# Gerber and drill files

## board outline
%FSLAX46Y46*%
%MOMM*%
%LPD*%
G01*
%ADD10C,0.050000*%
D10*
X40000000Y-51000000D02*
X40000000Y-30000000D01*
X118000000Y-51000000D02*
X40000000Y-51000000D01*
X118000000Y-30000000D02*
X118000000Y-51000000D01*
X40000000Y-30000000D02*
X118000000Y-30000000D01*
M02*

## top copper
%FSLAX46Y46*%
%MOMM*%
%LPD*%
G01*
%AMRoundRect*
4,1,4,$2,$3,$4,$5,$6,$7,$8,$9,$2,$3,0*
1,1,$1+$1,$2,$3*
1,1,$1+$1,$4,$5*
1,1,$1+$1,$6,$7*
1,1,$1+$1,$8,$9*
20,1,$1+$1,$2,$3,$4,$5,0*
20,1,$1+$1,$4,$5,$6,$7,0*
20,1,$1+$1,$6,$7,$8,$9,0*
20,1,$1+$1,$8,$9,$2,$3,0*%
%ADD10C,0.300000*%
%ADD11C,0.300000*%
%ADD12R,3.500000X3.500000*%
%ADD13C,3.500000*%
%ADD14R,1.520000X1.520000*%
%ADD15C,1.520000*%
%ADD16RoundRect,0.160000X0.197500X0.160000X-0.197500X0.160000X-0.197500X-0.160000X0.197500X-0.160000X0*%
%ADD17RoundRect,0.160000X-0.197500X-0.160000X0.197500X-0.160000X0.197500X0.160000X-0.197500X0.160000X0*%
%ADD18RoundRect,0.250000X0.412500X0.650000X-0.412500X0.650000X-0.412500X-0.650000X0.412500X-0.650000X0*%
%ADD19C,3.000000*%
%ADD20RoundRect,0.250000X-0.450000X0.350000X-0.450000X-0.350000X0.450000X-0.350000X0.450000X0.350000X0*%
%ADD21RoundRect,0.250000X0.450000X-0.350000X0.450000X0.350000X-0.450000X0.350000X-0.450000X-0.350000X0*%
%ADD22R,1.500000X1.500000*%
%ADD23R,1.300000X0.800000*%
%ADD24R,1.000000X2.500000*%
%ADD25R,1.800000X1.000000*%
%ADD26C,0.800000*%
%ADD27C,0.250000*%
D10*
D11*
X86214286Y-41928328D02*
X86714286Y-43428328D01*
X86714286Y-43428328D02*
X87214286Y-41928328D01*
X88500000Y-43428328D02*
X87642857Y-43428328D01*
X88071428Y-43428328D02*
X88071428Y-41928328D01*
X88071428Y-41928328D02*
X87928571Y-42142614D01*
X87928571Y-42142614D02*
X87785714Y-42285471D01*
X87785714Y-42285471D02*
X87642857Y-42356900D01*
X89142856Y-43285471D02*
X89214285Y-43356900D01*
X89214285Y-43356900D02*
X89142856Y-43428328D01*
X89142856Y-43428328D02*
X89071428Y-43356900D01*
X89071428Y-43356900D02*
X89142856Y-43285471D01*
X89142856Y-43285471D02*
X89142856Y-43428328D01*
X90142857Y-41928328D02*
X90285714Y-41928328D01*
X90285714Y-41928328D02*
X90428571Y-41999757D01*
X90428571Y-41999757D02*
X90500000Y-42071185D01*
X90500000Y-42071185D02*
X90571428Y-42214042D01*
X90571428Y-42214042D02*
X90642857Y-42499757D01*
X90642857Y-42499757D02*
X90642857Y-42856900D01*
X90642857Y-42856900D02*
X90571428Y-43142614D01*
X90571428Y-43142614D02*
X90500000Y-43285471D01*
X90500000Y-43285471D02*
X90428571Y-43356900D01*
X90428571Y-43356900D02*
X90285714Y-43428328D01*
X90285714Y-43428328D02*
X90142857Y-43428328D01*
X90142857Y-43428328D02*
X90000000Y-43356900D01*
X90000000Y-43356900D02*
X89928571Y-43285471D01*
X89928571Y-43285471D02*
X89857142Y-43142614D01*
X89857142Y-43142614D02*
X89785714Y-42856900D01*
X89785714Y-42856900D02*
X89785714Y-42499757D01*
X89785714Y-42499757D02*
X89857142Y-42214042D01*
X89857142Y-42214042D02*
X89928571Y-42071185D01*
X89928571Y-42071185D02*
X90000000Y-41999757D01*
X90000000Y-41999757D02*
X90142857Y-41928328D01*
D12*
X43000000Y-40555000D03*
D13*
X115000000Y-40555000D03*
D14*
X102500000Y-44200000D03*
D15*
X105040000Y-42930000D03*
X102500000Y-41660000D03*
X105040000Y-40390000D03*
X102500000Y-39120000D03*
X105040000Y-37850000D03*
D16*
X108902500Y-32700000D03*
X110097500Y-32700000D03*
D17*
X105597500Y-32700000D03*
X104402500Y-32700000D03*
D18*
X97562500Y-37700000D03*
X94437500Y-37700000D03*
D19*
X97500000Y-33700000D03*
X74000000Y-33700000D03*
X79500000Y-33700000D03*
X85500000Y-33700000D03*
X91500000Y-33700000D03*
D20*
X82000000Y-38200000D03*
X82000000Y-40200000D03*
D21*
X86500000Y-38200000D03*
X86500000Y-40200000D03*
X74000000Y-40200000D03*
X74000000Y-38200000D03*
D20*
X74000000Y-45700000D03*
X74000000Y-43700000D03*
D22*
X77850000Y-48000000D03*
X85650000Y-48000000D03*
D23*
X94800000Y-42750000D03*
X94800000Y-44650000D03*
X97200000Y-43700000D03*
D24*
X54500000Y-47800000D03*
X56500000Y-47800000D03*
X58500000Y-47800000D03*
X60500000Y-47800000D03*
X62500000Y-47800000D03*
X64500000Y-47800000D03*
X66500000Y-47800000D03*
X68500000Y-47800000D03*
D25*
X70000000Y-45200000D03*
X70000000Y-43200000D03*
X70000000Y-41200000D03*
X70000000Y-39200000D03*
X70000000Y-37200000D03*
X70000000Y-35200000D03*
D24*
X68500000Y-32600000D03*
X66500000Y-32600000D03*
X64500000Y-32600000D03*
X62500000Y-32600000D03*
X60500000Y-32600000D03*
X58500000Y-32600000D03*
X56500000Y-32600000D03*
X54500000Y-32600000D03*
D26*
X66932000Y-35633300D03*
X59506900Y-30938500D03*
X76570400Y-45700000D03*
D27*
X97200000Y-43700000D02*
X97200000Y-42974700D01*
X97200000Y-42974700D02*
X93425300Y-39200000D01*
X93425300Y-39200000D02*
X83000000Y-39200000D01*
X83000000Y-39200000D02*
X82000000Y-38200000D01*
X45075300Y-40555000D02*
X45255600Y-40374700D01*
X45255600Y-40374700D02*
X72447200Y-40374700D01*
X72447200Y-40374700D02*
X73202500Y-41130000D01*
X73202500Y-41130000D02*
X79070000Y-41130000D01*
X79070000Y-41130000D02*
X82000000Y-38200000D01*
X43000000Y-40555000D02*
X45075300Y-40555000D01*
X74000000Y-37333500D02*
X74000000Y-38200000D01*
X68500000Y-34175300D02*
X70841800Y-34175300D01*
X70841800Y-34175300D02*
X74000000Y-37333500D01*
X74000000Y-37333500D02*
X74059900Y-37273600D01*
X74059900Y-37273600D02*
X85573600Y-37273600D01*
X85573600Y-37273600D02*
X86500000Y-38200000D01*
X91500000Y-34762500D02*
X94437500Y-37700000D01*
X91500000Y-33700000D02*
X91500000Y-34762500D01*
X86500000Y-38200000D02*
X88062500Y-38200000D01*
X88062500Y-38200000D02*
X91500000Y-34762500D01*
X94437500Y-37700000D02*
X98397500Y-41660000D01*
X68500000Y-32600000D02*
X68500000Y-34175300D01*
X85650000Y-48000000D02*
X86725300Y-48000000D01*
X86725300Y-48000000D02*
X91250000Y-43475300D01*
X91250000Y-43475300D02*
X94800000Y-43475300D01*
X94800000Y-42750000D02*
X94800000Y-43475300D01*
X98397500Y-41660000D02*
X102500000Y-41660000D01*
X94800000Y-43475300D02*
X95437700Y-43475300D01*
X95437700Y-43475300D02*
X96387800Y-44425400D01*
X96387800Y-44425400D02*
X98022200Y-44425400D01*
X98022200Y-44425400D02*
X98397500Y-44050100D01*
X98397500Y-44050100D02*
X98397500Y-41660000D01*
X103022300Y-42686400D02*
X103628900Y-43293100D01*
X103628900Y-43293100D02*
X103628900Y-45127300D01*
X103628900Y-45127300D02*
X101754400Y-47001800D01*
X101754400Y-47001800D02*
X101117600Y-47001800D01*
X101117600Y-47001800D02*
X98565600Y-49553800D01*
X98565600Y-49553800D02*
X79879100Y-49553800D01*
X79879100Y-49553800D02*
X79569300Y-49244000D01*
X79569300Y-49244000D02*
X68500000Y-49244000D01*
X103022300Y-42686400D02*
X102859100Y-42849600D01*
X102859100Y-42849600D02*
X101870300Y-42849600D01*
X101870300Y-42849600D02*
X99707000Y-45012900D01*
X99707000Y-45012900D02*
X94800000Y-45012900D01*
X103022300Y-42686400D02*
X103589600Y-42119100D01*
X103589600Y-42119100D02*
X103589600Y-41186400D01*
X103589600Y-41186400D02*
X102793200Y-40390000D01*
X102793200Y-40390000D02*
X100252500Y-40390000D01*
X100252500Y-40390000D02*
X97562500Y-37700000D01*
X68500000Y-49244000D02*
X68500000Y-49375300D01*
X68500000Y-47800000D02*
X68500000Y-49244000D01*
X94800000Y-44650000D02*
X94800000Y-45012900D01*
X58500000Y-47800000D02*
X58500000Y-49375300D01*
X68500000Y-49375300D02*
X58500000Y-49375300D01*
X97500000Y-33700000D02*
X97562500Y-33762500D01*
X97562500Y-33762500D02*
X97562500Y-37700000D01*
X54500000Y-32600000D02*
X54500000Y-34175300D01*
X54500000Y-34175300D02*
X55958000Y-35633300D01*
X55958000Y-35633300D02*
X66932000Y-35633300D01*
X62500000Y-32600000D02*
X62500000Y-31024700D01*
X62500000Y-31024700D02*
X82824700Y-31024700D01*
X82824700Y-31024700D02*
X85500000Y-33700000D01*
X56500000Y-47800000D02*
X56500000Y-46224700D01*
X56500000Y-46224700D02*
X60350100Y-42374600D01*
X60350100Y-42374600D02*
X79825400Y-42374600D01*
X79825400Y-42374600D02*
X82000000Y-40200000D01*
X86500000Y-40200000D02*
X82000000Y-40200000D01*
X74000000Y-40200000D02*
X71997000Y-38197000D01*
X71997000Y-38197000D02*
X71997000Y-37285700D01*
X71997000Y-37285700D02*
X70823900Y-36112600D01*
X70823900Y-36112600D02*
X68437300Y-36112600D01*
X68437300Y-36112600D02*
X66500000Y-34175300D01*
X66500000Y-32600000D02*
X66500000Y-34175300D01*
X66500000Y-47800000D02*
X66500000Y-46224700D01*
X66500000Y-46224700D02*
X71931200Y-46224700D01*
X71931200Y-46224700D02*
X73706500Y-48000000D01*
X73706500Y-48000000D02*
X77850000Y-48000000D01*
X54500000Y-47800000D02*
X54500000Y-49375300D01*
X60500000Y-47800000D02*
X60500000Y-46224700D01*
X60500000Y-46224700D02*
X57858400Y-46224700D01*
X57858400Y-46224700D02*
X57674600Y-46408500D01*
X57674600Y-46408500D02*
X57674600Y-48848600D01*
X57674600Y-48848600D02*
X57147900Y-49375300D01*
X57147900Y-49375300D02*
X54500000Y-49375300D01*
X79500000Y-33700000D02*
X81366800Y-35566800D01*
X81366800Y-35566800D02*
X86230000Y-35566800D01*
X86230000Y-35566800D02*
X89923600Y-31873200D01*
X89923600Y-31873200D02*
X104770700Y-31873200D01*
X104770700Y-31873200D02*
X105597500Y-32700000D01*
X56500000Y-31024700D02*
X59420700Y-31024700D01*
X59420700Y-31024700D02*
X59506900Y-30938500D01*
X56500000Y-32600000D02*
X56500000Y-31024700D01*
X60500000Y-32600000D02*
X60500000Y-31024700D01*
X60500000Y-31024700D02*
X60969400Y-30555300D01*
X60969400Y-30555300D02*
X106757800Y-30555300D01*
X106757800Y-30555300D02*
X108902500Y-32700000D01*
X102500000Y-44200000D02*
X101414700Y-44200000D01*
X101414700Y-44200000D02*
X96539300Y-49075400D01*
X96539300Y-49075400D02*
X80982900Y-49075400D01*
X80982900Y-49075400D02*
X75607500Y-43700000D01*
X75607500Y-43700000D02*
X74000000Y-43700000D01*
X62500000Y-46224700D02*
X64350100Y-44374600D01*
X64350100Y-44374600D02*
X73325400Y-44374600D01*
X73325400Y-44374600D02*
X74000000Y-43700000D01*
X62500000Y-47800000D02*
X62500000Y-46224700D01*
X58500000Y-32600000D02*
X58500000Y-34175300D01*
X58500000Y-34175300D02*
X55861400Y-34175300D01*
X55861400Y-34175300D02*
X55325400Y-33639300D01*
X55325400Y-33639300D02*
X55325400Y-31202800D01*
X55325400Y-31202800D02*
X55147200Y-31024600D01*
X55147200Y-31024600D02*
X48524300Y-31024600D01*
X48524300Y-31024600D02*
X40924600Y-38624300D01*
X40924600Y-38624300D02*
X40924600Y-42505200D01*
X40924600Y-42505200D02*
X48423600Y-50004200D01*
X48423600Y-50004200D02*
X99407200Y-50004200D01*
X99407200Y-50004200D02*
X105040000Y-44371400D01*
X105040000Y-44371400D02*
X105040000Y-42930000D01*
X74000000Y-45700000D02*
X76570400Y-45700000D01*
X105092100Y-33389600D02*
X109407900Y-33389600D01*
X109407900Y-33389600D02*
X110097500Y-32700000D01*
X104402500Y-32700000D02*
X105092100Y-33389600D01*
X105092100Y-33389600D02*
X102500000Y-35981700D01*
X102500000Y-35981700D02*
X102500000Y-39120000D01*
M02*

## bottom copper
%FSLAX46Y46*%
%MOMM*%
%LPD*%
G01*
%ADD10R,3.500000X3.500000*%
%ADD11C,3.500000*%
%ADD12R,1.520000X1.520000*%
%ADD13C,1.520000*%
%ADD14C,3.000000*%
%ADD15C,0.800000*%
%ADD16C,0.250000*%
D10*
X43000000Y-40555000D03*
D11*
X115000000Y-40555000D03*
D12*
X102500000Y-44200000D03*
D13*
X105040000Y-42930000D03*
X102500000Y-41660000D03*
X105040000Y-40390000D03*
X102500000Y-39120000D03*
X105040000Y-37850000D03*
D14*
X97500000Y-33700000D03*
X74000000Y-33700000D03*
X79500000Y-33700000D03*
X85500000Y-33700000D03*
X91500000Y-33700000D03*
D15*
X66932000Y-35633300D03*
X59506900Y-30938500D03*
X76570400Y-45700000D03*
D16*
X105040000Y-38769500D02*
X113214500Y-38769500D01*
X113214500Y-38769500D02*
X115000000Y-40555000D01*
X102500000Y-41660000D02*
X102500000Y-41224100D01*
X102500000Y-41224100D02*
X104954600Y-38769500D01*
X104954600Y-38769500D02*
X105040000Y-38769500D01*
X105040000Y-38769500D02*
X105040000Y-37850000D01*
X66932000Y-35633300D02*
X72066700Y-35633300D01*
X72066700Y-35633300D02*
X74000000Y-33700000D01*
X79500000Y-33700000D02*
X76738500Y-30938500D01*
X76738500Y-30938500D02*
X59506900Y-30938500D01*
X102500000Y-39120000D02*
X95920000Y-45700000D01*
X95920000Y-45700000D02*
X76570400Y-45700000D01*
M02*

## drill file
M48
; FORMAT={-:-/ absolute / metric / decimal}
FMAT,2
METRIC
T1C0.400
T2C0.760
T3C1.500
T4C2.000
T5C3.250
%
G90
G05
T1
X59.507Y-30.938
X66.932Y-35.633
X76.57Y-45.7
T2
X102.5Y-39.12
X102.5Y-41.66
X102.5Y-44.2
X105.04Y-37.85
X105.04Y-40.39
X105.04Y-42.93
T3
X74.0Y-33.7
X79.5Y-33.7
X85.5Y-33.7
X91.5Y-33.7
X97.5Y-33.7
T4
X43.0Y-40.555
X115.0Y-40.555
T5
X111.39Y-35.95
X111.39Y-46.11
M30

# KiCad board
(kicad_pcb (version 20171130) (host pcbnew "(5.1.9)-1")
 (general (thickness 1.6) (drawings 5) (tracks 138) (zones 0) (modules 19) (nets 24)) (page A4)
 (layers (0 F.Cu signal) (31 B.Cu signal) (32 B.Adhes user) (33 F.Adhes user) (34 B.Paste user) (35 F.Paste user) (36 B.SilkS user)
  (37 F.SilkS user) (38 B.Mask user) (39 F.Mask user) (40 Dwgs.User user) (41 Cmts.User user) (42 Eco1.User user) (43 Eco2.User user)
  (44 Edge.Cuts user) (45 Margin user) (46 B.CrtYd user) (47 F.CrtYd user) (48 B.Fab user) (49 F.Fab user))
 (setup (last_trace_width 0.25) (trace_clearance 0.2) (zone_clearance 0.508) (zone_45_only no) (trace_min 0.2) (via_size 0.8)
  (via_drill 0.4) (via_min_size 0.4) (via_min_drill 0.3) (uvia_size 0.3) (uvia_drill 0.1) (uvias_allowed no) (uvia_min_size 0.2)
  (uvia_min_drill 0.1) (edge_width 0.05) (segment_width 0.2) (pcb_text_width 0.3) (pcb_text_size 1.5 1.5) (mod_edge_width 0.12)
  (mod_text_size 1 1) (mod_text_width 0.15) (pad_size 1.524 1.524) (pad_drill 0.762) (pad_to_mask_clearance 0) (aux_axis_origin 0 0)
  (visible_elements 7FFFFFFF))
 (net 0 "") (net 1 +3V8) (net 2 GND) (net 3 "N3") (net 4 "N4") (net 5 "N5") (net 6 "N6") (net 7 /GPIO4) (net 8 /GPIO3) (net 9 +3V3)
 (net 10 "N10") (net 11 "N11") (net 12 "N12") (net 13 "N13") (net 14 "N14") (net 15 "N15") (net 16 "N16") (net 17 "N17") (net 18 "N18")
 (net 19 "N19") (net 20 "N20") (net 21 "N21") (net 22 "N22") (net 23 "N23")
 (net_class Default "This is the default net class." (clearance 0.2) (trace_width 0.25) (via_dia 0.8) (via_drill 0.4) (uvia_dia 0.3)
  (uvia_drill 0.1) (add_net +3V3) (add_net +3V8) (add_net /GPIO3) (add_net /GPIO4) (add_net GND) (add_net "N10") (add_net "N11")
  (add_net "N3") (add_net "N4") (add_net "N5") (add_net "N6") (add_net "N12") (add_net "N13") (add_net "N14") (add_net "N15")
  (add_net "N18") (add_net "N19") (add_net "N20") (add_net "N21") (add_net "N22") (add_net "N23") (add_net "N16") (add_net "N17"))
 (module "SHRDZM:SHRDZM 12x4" (layer F.Cu) (at 93.5 47.75)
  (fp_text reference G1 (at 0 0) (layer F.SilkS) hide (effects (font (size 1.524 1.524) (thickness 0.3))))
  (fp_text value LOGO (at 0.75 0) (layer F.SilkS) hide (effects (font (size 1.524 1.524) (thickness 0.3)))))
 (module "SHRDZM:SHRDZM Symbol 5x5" (layer F.Cu) (at 43 34.75)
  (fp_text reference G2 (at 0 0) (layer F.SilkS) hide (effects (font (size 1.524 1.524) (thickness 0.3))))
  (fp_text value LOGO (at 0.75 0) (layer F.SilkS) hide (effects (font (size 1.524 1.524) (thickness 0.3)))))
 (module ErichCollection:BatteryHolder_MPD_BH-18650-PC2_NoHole (layer B.Cu) (at 43 40.555)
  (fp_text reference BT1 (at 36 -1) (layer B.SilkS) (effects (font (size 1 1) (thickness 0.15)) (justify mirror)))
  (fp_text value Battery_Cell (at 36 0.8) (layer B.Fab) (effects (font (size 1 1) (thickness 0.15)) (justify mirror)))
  (pad 1 thru_hole rect (at 0 0) (size 3.5 3.5) (drill 2) (layers *.Cu *.Mask) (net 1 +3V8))
  (pad 2 thru_hole circle (at 72 0) (size 3.5 3.5) (drill 2) (layers *.Cu *.Mask) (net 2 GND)))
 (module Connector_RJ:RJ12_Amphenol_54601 (layer F.Cu) (at 102.5 44.2 90)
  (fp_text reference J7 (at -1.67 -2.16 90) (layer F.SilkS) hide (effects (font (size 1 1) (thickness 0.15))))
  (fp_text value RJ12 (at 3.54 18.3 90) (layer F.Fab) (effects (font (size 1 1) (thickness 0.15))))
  (pad 1 thru_hole rect (at 0 0 90) (size 1.52 1.52) (drill 0.76) (layers *.Cu *.Mask) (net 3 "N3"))
  (pad "" np_thru_hole circle (at -1.91 8.89 90) (size 3.25 3.25) (drill 3.25) (layers *.Cu *.Mask))
  (pad 2 thru_hole circle (at 1.27 2.54 90) (size 1.52 1.52) (drill 0.76) (layers *.Cu *.Mask) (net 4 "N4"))
  (pad 3 thru_hole circle (at 2.54 0 90) (size 1.52 1.52) (drill 0.76) (layers *.Cu *.Mask) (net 2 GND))
  (pad 4 thru_hole circle (at 3.81 2.54 90) (size 1.52 1.52) (drill 0.76) (layers *.Cu *.Mask) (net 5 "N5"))
  (pad 5 thru_hole circle (at 5.08 0 90) (size 1.52 1.52) (drill 0.76) (layers *.Cu *.Mask) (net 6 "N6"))
  (pad 6 thru_hole circle (at 6.35 2.54 90) (size 1.52 1.52) (drill 0.76) (layers *.Cu *.Mask) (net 2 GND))
  (pad "" np_thru_hole circle (at 8.25 8.89 90) (size 3.25 3.25) (drill 3.25) (layers *.Cu *.Mask)))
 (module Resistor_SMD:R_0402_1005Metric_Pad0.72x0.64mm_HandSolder (layer F.Cu) (at 109.5 32.7 180)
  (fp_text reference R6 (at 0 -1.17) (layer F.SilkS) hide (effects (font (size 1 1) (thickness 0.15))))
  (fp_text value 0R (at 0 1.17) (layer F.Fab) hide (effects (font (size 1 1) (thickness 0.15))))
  (pad 2 smd roundrect (at 0.5975 0 180) (size 0.715 0.64) (layers F.Cu F.Paste F.Mask) (roundrect_rratio 0.25) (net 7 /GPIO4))
  (pad 1 smd roundrect (at -0.5975 0 180) (size 0.715 0.64) (layers F.Cu F.Paste F.Mask) (roundrect_rratio 0.25) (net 6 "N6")))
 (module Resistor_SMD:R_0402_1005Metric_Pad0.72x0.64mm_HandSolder (layer F.Cu) (at 105 32.7)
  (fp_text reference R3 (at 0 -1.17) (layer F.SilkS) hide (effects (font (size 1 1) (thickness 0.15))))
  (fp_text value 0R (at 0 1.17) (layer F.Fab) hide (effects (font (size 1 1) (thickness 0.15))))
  (pad 2 smd roundrect (at 0.5975 0) (size 0.715 0.64) (layers F.Cu F.Paste F.Mask) (roundrect_rratio 0.25) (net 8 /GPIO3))
  (pad 1 smd roundrect (at -0.5975 0) (size 0.715 0.64) (layers F.Cu F.Paste F.Mask) (roundrect_rratio 0.25) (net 6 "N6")))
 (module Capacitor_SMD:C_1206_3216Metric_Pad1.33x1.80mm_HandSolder (layer F.Cu) (at 96 37.7 180)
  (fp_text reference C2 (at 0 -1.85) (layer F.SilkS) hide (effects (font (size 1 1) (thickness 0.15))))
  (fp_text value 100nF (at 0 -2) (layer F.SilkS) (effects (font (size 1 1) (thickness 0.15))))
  (pad 1 smd roundrect (at -1.5625 0 180) (size 1.325 1.8) (layers F.Cu F.Paste F.Mask) (roundrect_rratio 0.188679) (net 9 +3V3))
  (pad 2 smd roundrect (at 1.5625 0 180) (size 1.325 1.8) (layers F.Cu F.Paste F.Mask) (roundrect_rratio 0.188679) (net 2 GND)))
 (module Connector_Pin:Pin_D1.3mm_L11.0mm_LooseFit (layer F.Cu) (at 97.5 33.7)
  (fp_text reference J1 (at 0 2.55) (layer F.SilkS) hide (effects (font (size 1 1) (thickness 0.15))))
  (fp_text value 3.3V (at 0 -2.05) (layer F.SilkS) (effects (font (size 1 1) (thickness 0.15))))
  (pad 1 thru_hole circle (at 0 0) (size 3 3) (drill 1.5) (layers *.Cu *.Mask) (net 9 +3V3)))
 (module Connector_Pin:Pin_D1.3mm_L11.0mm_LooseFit (layer F.Cu) (at 74 33.7)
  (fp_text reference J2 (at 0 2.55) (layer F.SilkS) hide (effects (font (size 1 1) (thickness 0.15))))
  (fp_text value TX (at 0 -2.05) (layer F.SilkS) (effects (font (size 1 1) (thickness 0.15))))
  (pad 1 thru_hole circle (at 0 0) (size 3 3) (drill 1.5) (layers *.Cu *.Mask) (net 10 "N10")))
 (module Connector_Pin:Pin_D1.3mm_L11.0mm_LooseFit (layer F.Cu) (at 79.5 33.7)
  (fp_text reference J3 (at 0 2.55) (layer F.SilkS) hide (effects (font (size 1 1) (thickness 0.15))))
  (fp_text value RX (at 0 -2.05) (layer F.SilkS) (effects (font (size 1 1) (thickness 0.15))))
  (pad 1 thru_hole circle (at 0 0) (size 3 3) (drill 1.5) (layers *.Cu *.Mask) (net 8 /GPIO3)))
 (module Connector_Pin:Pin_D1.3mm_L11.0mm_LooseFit (layer F.Cu) (at 85.5 33.7)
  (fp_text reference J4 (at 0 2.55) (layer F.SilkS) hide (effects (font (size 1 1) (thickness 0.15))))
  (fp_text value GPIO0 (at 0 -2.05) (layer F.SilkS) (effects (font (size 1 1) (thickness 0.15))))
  (pad 1 thru_hole circle (at 0 0) (size 3 3) (drill 1.5) (layers *.Cu *.Mask) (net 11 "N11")))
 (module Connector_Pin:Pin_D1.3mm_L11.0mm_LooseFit (layer F.Cu) (at 91.5 33.7)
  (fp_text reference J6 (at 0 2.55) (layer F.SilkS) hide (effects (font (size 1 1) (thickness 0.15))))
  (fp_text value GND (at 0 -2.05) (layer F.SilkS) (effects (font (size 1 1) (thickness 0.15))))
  (pad 1 thru_hole circle (at 0 0) (size 3 3) (drill 1.5) (layers *.Cu *.Mask) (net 2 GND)))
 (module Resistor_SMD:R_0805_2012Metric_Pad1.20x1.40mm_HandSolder (layer F.Cu) (at 82 39.2 270)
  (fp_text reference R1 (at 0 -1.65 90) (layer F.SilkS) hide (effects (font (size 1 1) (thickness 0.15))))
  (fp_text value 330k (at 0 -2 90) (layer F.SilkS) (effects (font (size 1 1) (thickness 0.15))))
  (pad 1 smd roundrect (at -1 0 270) (size 1.2 1.4) (layers F.Cu F.Paste F.Mask) (roundrect_rratio 0.208333) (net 1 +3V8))
  (pad 2 smd roundrect (at 1 0 270) (size 1.2 1.4) (layers F.Cu F.Paste F.Mask) (roundrect_rratio 0.208333) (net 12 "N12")))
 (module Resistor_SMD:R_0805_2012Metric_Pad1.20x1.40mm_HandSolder (layer F.Cu) (at 86.5 39.2 90)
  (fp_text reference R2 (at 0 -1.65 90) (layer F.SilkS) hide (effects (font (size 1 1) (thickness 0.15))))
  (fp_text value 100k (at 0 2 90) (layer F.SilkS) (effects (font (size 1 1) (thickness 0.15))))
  (pad 2 smd roundrect (at 1 0 90) (size 1.2 1.4) (layers F.Cu F.Paste F.Mask) (roundrect_rratio 0.208333) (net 2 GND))
  (pad 1 smd roundrect (at -1 0 90) (size 1.2 1.4) (layers F.Cu F.Paste F.Mask) (roundrect_rratio 0.208333) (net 12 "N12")))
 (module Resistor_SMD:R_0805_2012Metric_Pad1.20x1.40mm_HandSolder (layer F.Cu) (at 74 39.2 90)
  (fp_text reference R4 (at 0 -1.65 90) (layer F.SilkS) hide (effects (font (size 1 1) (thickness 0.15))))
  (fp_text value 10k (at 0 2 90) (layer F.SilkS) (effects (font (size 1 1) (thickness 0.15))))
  (pad 1 smd roundrect (at -1 0 90) (size 1.2 1.4) (layers F.Cu F.Paste F.Mask) (roundrect_rratio 0.208333) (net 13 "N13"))
  (pad 2 smd roundrect (at 1 0 90) (size 1.2 1.4) (layers F.Cu F.Paste F.Mask) (roundrect_rratio 0.208333) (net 2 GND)))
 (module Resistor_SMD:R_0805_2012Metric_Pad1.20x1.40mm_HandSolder (layer F.Cu) (at 74 44.7 270)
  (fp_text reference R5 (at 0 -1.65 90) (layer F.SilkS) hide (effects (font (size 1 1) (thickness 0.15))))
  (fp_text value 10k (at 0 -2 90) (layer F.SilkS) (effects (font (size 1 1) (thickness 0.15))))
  (pad 2 smd roundrect (at 1 0 270) (size 1.2 1.4) (layers F.Cu F.Paste F.Mask) (roundrect_rratio 0.208333) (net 6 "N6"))
  (pad 1 smd roundrect (at -1 0 270) (size 1.2 1.4) (layers F.Cu F.Paste F.Mask) (roundrect_rratio 0.208333) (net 3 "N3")))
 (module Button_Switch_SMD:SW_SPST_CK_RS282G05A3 (layer F.Cu) (at 81.75 48)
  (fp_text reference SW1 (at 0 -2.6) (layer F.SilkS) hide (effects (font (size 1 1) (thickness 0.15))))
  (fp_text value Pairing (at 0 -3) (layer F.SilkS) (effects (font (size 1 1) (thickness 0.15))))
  (pad 1 smd rect (at -3.9 0) (size 1.5 1.5) (layers F.Cu F.Paste F.Mask) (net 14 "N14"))
  (pad 2 smd rect (at 3.9 0) (size 1.5 1.5) (layers F.Cu F.Paste F.Mask) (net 2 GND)))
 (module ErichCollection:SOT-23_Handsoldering (layer F.Cu) (at 96 43.7)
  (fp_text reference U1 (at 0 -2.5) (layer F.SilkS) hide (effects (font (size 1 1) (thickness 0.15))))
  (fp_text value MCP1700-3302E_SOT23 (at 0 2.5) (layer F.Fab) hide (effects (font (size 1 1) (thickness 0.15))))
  (pad 1 smd rect (at -1.2 -0.95) (size 1.3 0.8) (layers F.Cu F.Paste F.Mask) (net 2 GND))
  (pad 2 smd rect (at -1.2 0.95) (size 1.3 0.8) (layers F.Cu F.Paste F.Mask) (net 9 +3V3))
  (pad 3 smd rect (at 1.2 0) (size 1.3 0.8) (layers F.Cu F.Paste F.Mask) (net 1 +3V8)))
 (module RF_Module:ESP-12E (layer F.Cu) (at 58 40.2 90)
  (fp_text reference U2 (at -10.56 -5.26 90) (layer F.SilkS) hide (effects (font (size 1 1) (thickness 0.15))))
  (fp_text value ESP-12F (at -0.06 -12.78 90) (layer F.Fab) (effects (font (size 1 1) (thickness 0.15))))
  (pad 1 smd rect (at -7.6 -3.5 90) (size 2.5 1) (layers F.Cu F.Paste F.Mask) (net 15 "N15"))
  (pad 2 smd rect (at -7.6 -1.5 90) (size 2.5 1) (layers F.Cu F.Paste F.Mask) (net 12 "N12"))
  (pad 3 smd rect (at -7.6 0.5 90) (size 2.5 1) (layers F.Cu F.Paste F.Mask) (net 9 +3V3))
  (pad 4 smd rect (at -7.6 2.5 90) (size 2.5 1) (layers F.Cu F.Paste F.Mask) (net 15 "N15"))
  (pad 5 smd rect (at -7.6 4.5 90) (size 2.5 1) (layers F.Cu F.Paste F.Mask) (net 3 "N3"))
  (pad 6 smd rect (at -7.6 6.5 90) (size 2.5 1) (layers F.Cu F.Paste F.Mask) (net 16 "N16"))
  (pad 7 smd rect (at -7.6 8.5 90) (size 2.5 1) (layers F.Cu F.Paste F.Mask) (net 14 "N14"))
  (pad 8 smd rect (at -7.6 10.5 90) (size 2.5 1) (layers F.Cu F.Paste F.Mask) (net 9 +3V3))
  (pad 9 smd rect (at -5 12 90) (size 1 1.8) (layers F.Cu F.Paste F.Mask) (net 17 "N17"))
  (pad 10 smd rect (at -3 12 90) (size 1 1.8) (layers F.Cu F.Paste F.Mask) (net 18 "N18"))
  (pad 11 smd rect (at -1 12 90) (size 1 1.8) (layers F.Cu F.Paste F.Mask) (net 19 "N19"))
  (pad 12 smd rect (at 1 12 90) (size 1 1.8) (layers F.Cu F.Paste F.Mask) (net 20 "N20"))
  (pad 13 smd rect (at 3 12 90) (size 1 1.8) (layers F.Cu F.Paste F.Mask) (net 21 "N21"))
  (pad 14 smd rect (at 5 12 90) (size 1 1.8) (layers F.Cu F.Paste F.Mask) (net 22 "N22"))
  (pad 15 smd rect (at 7.6 10.5 90) (size 2.5 1) (layers F.Cu F.Paste F.Mask) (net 2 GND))
  (pad 16 smd rect (at 7.6 8.5 90) (size 2.5 1) (layers F.Cu F.Paste F.Mask) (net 13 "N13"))
  (pad 17 smd rect (at 7.6 6.5 90) (size 2.5 1) (layers F.Cu F.Paste F.Mask) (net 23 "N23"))
  (pad 18 smd rect (at 7.6 4.5 90) (size 2.5 1) (layers F.Cu F.Paste F.Mask) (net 11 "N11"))
  (pad 19 smd rect (at 7.6 2.5 90) (size 2.5 1) (layers F.Cu F.Paste F.Mask) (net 7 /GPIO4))
  (pad 20 smd rect (at 7.6 0.5 90) (size 2.5 1) (layers F.Cu F.Paste F.Mask) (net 4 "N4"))
  (pad 21 smd rect (at 7.6 -1.5 90) (size 2.5 1) (layers F.Cu F.Paste F.Mask) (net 8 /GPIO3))
  (pad 22 smd rect (at 7.6 -3.5 90) (size 2.5 1) (layers F.Cu F.Paste F.Mask) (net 10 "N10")))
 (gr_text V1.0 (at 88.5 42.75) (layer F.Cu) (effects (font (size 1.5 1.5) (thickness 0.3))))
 (gr_line (start 40 51) (end 40 30) (layer Edge.Cuts) (width 0.05))
 (gr_line (start 118 51) (end 40 51) (layer Edge.Cuts) (width 0.05))
 (gr_line (start 118 30) (end 118 51) (layer Edge.Cuts) (width 0.05))
 (gr_line (start 40 30) (end 118 30) (layer Edge.Cuts) (width 0.05))
 (segment (start 97.2 43.7) (end 97.2 42.9747) (width 0.25) (layer F.Cu) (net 1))
 (segment (start 97.2 42.9747) (end 93.4253 39.2) (width 0.25) (layer F.Cu) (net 1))
 (segment (start 93.4253 39.2) (end 83 39.2) (width 0.25) (layer F.Cu) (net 1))
 (segment (start 83 39.2) (end 82 38.2) (width 0.25) (layer F.Cu) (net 1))
 (segment (start 45.0753 40.555) (end 45.2556 40.3747) (width 0.25) (layer F.Cu) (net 1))
 (segment (start 45.2556 40.3747) (end 72.4472 40.3747) (width 0.25) (layer F.Cu) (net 1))
 (segment (start 72.4472 40.3747) (end 73.2025 41.13) (width 0.25) (layer F.Cu) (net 1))
 (segment (start 73.2025 41.13) (end 79.07 41.13) (width 0.25) (layer F.Cu) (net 1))
 (segment (start 79.07 41.13) (end 82 38.2) (width 0.25) (layer F.Cu) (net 1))
 (segment (start 43 40.555) (end 45.0753 40.555) (width 0.25) (layer F.Cu) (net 1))
 (segment (start 74 37.3335) (end 74 38.2) (width 0.25) (layer F.Cu) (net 2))
 (segment (start 68.5 34.1753) (end 70.8418 34.1753) (width 0.25) (layer F.Cu) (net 2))
 (segment (start 70.8418 34.1753) (end 74 37.3335) (width 0.25) (layer F.Cu) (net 2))
 (segment (start 74 37.3335) (end 74.0599 37.2736) (width 0.25) (layer F.Cu) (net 2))
 (segment (start 74.0599 37.2736) (end 85.5736 37.2736) (width 0.25) (layer F.Cu) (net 2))
 (segment (start 85.5736 37.2736) (end 86.5 38.2) (width 0.25) (layer F.Cu) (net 2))
 (segment (start 91.5 34.7625) (end 94.4375 37.7) (width 0.25) (layer F.Cu) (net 2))
 (segment (start 91.5 33.7) (end 91.5 34.7625) (width 0.25) (layer F.Cu) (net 2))
 (segment (start 86.5 38.2) (end 88.0625 38.2) (width 0.25) (layer F.Cu) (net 2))
 (segment (start 88.0625 38.2) (end 91.5 34.7625) (width 0.25) (layer F.Cu) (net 2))
 (segment (start 94.4375 37.7) (end 98.3975 41.66) (width 0.25) (layer F.Cu) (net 2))
 (segment (start 68.5 32.6) (end 68.5 34.1753) (width 0.25) (layer F.Cu) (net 2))
 (segment (start 85.65 48) (end 86.7253 48) (width 0.25) (layer F.Cu) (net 2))
 (segment (start 86.7253 48) (end 91.25 43.4753) (width 0.25) (layer F.Cu) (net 2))
 (segment (start 91.25 43.4753) (end 94.8 43.4753) (width 0.25) (layer F.Cu) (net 2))
 (segment (start 94.8 42.75) (end 94.8 43.4753) (width 0.25) (layer F.Cu) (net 2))
 (segment (start 98.3975 41.66) (end 102.5 41.66) (width 0.25) (layer F.Cu) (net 2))
 (segment (start 94.8 43.4753) (end 95.4377 43.4753) (width 0.25) (layer F.Cu) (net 2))
 (segment (start 95.4377 43.4753) (end 96.3878 44.4254) (width 0.25) (layer F.Cu) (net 2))
 (segment (start 96.3878 44.4254) (end 98.0222 44.4254) (width 0.25) (layer F.Cu) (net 2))
 (segment (start 98.0222 44.4254) (end 98.3975 44.0501) (width 0.25) (layer F.Cu) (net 2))
 (segment (start 98.3975 44.0501) (end 98.3975 41.66) (width 0.25) (layer F.Cu) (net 2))
 (segment (start 105.04 38.7695) (end 113.2145 38.7695) (width 0.25) (layer B.Cu) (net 2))
 (segment (start 113.2145 38.7695) (end 115 40.555) (width 0.25) (layer B.Cu) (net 2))
 (segment (start 102.5 41.66) (end 102.5 41.2241) (width 0.25) (layer B.Cu) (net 2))
 (segment (start 102.5 41.2241) (end 104.9546 38.7695) (width 0.25) (layer B.Cu) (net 2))
 (segment (start 104.9546 38.7695) (end 105.04 38.7695) (width 0.25) (layer B.Cu) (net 2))
 (segment (start 105.04 38.7695) (end 105.04 37.85) (width 0.25) (layer B.Cu) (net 2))
 (segment (start 103.0223 42.6864) (end 103.6289 43.2931) (width 0.25) (layer F.Cu) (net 9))
 (segment (start 103.6289 43.2931) (end 103.6289 45.1273) (width 0.25) (layer F.Cu) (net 9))
 (segment (start 103.6289 45.1273) (end 101.7544 47.0018) (width 0.25) (layer F.Cu) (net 9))
 (segment (start 101.7544 47.0018) (end 101.1176 47.0018) (width 0.25) (layer F.Cu) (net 9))
 (segment (start 101.1176 47.0018) (end 98.5656 49.5538) (width 0.25) (layer F.Cu) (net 9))
 (segment (start 98.5656 49.5538) (end 79.8791 49.5538) (width 0.25) (layer F.Cu) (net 9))
 (segment (start 79.8791 49.5538) (end 79.5693 49.244) (width 0.25) (layer F.Cu) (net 9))
 (segment (start 79.5693 49.244) (end 68.5 49.244) (width 0.25) (layer F.Cu) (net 9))
 (segment (start 103.0223 42.6864) (end 102.8591 42.8496) (width 0.25) (layer F.Cu) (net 9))
 (segment (start 102.8591 42.8496) (end 101.8703 42.8496) (width 0.25) (layer F.Cu) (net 9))
 (segment (start 101.8703 42.8496) (end 99.707 45.0129) (width 0.25) (layer F.Cu) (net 9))
 (segment (start 99.707 45.0129) (end 94.8 45.0129) (width 0.25) (layer F.Cu) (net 9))
 (segment (start 103.0223 42.6864) (end 103.5896 42.1191) (width 0.25) (layer F.Cu) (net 9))
 (segment (start 103.5896 42.1191) (end 103.5896 41.1864) (width 0.25) (layer F.Cu) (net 9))
 (segment (start 103.5896 41.1864) (end 102.7932 40.39) (width 0.25) (layer F.Cu) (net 9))
 (segment (start 102.7932 40.39) (end 100.2525 40.39) (width 0.25) (layer F.Cu) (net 9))
 (segment (start 100.2525 40.39) (end 97.5625 37.7) (width 0.25) (layer F.Cu) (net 9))
 (segment (start 68.5 49.244) (end 68.5 49.3753) (width 0.25) (layer F.Cu) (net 9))
 (segment (start 68.5 47.8) (end 68.5 49.244) (width 0.25) (layer F.Cu) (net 9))
 (segment (start 94.8 44.65) (end 94.8 45.0129) (width 0.25) (layer F.Cu) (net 9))
 (segment (start 58.5 47.8) (end 58.5 49.3753) (width 0.25) (layer F.Cu) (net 9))
 (segment (start 68.5 49.3753) (end 58.5 49.3753) (width 0.25) (layer F.Cu) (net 9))
 (segment (start 97.5 33.7) (end 97.5625 33.7625) (width 0.25) (layer F.Cu) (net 9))
 (segment (start 97.5625 33.7625) (end 97.5625 37.7) (width 0.25) (layer F.Cu) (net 9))
 (segment (start 54.5 32.6) (end 54.5 34.1753) (width 0.25) (layer F.Cu) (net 10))
 (segment (start 54.5 34.1753) (end 55.958 35.6333) (width 0.25) (layer F.Cu) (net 10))
 (segment (start 55.958 35.6333) (end 66.932 35.6333) (width 0.25) (layer F.Cu) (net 10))
 (segment (start 66.932 35.6333) (end 72.0667 35.6333) (width 0.25) (layer B.Cu) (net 10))
 (segment (start 72.0667 35.6333) (end 74 33.7) (width 0.25) (layer B.Cu) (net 10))
 (via (at 66.932 35.6333) (size 0.8) (layers F.Cu B.Cu) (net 10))
 (segment (start 62.5 32.6) (end 62.5 31.0247) (width 0.25) (layer F.Cu) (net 11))
 (segment (start 62.5 31.0247) (end 82.8247 31.0247) (width 0.25) (layer F.Cu) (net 11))
 (segment (start 82.8247 31.0247) (end 85.5 33.7) (width 0.25) (layer F.Cu) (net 11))
 (segment (start 56.5 47.8) (end 56.5 46.2247) (width 0.25) (layer F.Cu) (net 12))
 (segment (start 56.5 46.2247) (end 60.3501 42.3746) (width 0.25) (layer F.Cu) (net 12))
 (segment (start 60.3501 42.3746) (end 79.8254 42.3746) (width 0.25) (layer F.Cu) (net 12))
 (segment (start 79.8254 42.3746) (end 82 40.2) (width 0.25) (layer F.Cu) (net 12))
 (segment (start 86.5 40.2) (end 82 40.2) (width 0.25) (layer F.Cu) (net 12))
 (segment (start 74 40.2) (end 71.997 38.197) (width 0.25) (layer F.Cu) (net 13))
 (segment (start 71.997 38.197) (end 71.997 37.2857) (width 0.25) (layer F.Cu) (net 13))
 (segment (start 71.997 37.2857) (end 70.8239 36.1126) (width 0.25) (layer F.Cu) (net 13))
 (segment (start 70.8239 36.1126) (end 68.4373 36.1126) (width 0.25) (layer F.Cu) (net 13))
 (segment (start 68.4373 36.1126) (end 66.5 34.1753) (width 0.25) (layer F.Cu) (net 13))
 (segment (start 66.5 32.6) (end 66.5 34.1753) (width 0.25) (layer F.Cu) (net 13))
 (segment (start 66.5 47.8) (end 66.5 46.2247) (width 0.25) (layer F.Cu) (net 14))
 (segment (start 66.5 46.2247) (end 71.9312 46.2247) (width 0.25) (layer F.Cu) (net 14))
 (segment (start 71.9312 46.2247) (end 73.7065 48) (width 0.25) (layer F.Cu) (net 14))
 (segment (start 73.7065 48) (end 77.85 48) (width 0.25) (layer F.Cu) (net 14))
 (segment (start 54.5 47.8) (end 54.5 49.3753) (width 0.25) (layer F.Cu) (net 15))
 (segment (start 60.5 47.8) (end 60.5 46.2247) (width 0.25) (layer F.Cu) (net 15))
 (segment (start 60.5 46.2247) (end 57.8584 46.2247) (width 0.25) (layer F.Cu) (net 15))
 (segment (start 57.8584 46.2247) (end 57.6746 46.4085) (width 0.25) (layer F.Cu) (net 15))
 (segment (start 57.6746 46.4085) (end 57.6746 48.8486) (width 0.25) (layer F.Cu) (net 15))
 (segment (start 57.6746 48.8486) (end 57.1479 49.3753) (width 0.25) (layer F.Cu) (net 15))
 (segment (start 57.1479 49.3753) (end 54.5 49.3753) (width 0.25) (layer F.Cu) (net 15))
 (segment (start 79.5 33.7) (end 81.3668 35.5668) (width 0.25) (layer F.Cu) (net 8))
 (segment (start 81.3668 35.5668) (end 86.23 35.5668) (width 0.25) (layer F.Cu) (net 8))
 (segment (start 86.23 35.5668) (end 89.9236 31.8732) (width 0.25) (layer F.Cu) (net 8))
 (segment (start 89.9236 31.8732) (end 104.7707 31.8732) (width 0.25) (layer F.Cu) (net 8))
 (segment (start 104.7707 31.8732) (end 105.5975 32.7) (width 0.25) (layer F.Cu) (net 8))
 (segment (start 56.5 31.0247) (end 59.4207 31.0247) (width 0.25) (layer F.Cu) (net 8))
 (segment (start 59.4207 31.0247) (end 59.5069 30.9385) (width 0.25) (layer F.Cu) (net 8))
 (segment (start 79.5 33.7) (end 76.7385 30.9385) (width 0.25) (layer B.Cu) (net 8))
 (segment (start 76.7385 30.9385) (end 59.5069 30.9385) (width 0.25) (layer B.Cu) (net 8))
 (segment (start 56.5 32.6) (end 56.5 31.0247) (width 0.25) (layer F.Cu) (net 8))
 (via (at 59.5069 30.9385) (size 0.8) (layers F.Cu B.Cu) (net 8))
 (segment (start 60.5 32.6) (end 60.5 31.0247) (width 0.25) (layer F.Cu) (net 7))
 (segment (start 60.5 31.0247) (end 60.9694 30.5553) (width 0.25) (layer F.Cu) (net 7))
 (segment (start 60.9694 30.5553) (end 106.7578 30.5553) (width 0.25) (layer F.Cu) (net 7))
 (segment (start 106.7578 30.5553) (end 108.9025 32.7) (width 0.25) (layer F.Cu) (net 7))
 (segment (start 102.5 44.2) (end 101.4147 44.2) (width 0.25) (layer F.Cu) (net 3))
 (segment (start 101.4147 44.2) (end 96.5393 49.0754) (width 0.25) (layer F.Cu) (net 3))
 (segment (start 96.5393 49.0754) (end 80.9829 49.0754) (width 0.25) (layer F.Cu) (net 3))
 (segment (start 80.9829 49.0754) (end 75.6075 43.7) (width 0.25) (layer F.Cu) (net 3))
 (segment (start 75.6075 43.7) (end 74 43.7) (width 0.25) (layer F.Cu) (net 3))
 (segment (start 62.5 46.2247) (end 64.3501 44.3746) (width 0.25) (layer F.Cu) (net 3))
 (segment (start 64.3501 44.3746) (end 73.3254 44.3746) (width 0.25) (layer F.Cu) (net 3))
 (segment (start 73.3254 44.3746) (end 74 43.7) (width 0.25) (layer F.Cu) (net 3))
 (segment (start 62.5 47.8) (end 62.5 46.2247) (width 0.25) (layer F.Cu) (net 3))
 (segment (start 58.5 32.6) (end 58.5 34.1753) (width 0.25) (layer F.Cu) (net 4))
 (segment (start 58.5 34.1753) (end 55.8614 34.1753) (width 0.25) (layer F.Cu) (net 4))
 (segment (start 55.8614 34.1753) (end 55.3254 33.6393) (width 0.25) (layer F.Cu) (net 4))
 (segment (start 55.3254 33.6393) (end 55.3254 31.2028) (width 0.25) (layer F.Cu) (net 4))
 (segment (start 55.3254 31.2028) (end 55.1472 31.0246) (width 0.25) (layer F.Cu) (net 4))
 (segment (start 55.1472 31.0246) (end 48.5243 31.0246) (width 0.25) (layer F.Cu) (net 4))
 (segment (start 48.5243 31.0246) (end 40.9246 38.6243) (width 0.25) (layer F.Cu) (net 4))
 (segment (start 40.9246 38.6243) (end 40.9246 42.5052) (width 0.25) (layer F.Cu) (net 4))
 (segment (start 40.9246 42.5052) (end 48.4236 50.0042) (width 0.25) (layer F.Cu) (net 4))
 (segment (start 48.4236 50.0042) (end 99.4072 50.0042) (width 0.25) (layer F.Cu) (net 4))
 (segment (start 99.4072 50.0042) (end 105.04 44.3714) (width 0.25) (layer F.Cu) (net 4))
 (segment (start 105.04 44.3714) (end 105.04 42.93) (width 0.25) (layer F.Cu) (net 4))
 (segment (start 74 45.7) (end 76.5704 45.7) (width 0.25) (layer F.Cu) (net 6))
 (segment (start 102.5 39.12) (end 95.92 45.7) (width 0.25) (layer B.Cu) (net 6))
 (segment (start 95.92 45.7) (end 76.5704 45.7) (width 0.25) (layer B.Cu) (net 6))
 (segment (start 105.0921 33.3896) (end 109.4079 33.3896) (width 0.25) (layer F.Cu) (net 6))
 (segment (start 109.4079 33.3896) (end 110.0975 32.7) (width 0.25) (layer F.Cu) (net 6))
 (segment (start 104.4025 32.7) (end 105.0921 33.3896) (width 0.25) (layer F.Cu) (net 6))
 (segment (start 105.0921 33.3896) (end 102.5 35.9817) (width 0.25) (layer F.Cu) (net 6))
 (segment (start 102.5 35.9817) (end 102.5 39.12) (width 0.25) (layer F.Cu) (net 6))
 (via (at 76.5704 45.7) (size 0.8) (layers F.Cu B.Cu) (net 6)))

